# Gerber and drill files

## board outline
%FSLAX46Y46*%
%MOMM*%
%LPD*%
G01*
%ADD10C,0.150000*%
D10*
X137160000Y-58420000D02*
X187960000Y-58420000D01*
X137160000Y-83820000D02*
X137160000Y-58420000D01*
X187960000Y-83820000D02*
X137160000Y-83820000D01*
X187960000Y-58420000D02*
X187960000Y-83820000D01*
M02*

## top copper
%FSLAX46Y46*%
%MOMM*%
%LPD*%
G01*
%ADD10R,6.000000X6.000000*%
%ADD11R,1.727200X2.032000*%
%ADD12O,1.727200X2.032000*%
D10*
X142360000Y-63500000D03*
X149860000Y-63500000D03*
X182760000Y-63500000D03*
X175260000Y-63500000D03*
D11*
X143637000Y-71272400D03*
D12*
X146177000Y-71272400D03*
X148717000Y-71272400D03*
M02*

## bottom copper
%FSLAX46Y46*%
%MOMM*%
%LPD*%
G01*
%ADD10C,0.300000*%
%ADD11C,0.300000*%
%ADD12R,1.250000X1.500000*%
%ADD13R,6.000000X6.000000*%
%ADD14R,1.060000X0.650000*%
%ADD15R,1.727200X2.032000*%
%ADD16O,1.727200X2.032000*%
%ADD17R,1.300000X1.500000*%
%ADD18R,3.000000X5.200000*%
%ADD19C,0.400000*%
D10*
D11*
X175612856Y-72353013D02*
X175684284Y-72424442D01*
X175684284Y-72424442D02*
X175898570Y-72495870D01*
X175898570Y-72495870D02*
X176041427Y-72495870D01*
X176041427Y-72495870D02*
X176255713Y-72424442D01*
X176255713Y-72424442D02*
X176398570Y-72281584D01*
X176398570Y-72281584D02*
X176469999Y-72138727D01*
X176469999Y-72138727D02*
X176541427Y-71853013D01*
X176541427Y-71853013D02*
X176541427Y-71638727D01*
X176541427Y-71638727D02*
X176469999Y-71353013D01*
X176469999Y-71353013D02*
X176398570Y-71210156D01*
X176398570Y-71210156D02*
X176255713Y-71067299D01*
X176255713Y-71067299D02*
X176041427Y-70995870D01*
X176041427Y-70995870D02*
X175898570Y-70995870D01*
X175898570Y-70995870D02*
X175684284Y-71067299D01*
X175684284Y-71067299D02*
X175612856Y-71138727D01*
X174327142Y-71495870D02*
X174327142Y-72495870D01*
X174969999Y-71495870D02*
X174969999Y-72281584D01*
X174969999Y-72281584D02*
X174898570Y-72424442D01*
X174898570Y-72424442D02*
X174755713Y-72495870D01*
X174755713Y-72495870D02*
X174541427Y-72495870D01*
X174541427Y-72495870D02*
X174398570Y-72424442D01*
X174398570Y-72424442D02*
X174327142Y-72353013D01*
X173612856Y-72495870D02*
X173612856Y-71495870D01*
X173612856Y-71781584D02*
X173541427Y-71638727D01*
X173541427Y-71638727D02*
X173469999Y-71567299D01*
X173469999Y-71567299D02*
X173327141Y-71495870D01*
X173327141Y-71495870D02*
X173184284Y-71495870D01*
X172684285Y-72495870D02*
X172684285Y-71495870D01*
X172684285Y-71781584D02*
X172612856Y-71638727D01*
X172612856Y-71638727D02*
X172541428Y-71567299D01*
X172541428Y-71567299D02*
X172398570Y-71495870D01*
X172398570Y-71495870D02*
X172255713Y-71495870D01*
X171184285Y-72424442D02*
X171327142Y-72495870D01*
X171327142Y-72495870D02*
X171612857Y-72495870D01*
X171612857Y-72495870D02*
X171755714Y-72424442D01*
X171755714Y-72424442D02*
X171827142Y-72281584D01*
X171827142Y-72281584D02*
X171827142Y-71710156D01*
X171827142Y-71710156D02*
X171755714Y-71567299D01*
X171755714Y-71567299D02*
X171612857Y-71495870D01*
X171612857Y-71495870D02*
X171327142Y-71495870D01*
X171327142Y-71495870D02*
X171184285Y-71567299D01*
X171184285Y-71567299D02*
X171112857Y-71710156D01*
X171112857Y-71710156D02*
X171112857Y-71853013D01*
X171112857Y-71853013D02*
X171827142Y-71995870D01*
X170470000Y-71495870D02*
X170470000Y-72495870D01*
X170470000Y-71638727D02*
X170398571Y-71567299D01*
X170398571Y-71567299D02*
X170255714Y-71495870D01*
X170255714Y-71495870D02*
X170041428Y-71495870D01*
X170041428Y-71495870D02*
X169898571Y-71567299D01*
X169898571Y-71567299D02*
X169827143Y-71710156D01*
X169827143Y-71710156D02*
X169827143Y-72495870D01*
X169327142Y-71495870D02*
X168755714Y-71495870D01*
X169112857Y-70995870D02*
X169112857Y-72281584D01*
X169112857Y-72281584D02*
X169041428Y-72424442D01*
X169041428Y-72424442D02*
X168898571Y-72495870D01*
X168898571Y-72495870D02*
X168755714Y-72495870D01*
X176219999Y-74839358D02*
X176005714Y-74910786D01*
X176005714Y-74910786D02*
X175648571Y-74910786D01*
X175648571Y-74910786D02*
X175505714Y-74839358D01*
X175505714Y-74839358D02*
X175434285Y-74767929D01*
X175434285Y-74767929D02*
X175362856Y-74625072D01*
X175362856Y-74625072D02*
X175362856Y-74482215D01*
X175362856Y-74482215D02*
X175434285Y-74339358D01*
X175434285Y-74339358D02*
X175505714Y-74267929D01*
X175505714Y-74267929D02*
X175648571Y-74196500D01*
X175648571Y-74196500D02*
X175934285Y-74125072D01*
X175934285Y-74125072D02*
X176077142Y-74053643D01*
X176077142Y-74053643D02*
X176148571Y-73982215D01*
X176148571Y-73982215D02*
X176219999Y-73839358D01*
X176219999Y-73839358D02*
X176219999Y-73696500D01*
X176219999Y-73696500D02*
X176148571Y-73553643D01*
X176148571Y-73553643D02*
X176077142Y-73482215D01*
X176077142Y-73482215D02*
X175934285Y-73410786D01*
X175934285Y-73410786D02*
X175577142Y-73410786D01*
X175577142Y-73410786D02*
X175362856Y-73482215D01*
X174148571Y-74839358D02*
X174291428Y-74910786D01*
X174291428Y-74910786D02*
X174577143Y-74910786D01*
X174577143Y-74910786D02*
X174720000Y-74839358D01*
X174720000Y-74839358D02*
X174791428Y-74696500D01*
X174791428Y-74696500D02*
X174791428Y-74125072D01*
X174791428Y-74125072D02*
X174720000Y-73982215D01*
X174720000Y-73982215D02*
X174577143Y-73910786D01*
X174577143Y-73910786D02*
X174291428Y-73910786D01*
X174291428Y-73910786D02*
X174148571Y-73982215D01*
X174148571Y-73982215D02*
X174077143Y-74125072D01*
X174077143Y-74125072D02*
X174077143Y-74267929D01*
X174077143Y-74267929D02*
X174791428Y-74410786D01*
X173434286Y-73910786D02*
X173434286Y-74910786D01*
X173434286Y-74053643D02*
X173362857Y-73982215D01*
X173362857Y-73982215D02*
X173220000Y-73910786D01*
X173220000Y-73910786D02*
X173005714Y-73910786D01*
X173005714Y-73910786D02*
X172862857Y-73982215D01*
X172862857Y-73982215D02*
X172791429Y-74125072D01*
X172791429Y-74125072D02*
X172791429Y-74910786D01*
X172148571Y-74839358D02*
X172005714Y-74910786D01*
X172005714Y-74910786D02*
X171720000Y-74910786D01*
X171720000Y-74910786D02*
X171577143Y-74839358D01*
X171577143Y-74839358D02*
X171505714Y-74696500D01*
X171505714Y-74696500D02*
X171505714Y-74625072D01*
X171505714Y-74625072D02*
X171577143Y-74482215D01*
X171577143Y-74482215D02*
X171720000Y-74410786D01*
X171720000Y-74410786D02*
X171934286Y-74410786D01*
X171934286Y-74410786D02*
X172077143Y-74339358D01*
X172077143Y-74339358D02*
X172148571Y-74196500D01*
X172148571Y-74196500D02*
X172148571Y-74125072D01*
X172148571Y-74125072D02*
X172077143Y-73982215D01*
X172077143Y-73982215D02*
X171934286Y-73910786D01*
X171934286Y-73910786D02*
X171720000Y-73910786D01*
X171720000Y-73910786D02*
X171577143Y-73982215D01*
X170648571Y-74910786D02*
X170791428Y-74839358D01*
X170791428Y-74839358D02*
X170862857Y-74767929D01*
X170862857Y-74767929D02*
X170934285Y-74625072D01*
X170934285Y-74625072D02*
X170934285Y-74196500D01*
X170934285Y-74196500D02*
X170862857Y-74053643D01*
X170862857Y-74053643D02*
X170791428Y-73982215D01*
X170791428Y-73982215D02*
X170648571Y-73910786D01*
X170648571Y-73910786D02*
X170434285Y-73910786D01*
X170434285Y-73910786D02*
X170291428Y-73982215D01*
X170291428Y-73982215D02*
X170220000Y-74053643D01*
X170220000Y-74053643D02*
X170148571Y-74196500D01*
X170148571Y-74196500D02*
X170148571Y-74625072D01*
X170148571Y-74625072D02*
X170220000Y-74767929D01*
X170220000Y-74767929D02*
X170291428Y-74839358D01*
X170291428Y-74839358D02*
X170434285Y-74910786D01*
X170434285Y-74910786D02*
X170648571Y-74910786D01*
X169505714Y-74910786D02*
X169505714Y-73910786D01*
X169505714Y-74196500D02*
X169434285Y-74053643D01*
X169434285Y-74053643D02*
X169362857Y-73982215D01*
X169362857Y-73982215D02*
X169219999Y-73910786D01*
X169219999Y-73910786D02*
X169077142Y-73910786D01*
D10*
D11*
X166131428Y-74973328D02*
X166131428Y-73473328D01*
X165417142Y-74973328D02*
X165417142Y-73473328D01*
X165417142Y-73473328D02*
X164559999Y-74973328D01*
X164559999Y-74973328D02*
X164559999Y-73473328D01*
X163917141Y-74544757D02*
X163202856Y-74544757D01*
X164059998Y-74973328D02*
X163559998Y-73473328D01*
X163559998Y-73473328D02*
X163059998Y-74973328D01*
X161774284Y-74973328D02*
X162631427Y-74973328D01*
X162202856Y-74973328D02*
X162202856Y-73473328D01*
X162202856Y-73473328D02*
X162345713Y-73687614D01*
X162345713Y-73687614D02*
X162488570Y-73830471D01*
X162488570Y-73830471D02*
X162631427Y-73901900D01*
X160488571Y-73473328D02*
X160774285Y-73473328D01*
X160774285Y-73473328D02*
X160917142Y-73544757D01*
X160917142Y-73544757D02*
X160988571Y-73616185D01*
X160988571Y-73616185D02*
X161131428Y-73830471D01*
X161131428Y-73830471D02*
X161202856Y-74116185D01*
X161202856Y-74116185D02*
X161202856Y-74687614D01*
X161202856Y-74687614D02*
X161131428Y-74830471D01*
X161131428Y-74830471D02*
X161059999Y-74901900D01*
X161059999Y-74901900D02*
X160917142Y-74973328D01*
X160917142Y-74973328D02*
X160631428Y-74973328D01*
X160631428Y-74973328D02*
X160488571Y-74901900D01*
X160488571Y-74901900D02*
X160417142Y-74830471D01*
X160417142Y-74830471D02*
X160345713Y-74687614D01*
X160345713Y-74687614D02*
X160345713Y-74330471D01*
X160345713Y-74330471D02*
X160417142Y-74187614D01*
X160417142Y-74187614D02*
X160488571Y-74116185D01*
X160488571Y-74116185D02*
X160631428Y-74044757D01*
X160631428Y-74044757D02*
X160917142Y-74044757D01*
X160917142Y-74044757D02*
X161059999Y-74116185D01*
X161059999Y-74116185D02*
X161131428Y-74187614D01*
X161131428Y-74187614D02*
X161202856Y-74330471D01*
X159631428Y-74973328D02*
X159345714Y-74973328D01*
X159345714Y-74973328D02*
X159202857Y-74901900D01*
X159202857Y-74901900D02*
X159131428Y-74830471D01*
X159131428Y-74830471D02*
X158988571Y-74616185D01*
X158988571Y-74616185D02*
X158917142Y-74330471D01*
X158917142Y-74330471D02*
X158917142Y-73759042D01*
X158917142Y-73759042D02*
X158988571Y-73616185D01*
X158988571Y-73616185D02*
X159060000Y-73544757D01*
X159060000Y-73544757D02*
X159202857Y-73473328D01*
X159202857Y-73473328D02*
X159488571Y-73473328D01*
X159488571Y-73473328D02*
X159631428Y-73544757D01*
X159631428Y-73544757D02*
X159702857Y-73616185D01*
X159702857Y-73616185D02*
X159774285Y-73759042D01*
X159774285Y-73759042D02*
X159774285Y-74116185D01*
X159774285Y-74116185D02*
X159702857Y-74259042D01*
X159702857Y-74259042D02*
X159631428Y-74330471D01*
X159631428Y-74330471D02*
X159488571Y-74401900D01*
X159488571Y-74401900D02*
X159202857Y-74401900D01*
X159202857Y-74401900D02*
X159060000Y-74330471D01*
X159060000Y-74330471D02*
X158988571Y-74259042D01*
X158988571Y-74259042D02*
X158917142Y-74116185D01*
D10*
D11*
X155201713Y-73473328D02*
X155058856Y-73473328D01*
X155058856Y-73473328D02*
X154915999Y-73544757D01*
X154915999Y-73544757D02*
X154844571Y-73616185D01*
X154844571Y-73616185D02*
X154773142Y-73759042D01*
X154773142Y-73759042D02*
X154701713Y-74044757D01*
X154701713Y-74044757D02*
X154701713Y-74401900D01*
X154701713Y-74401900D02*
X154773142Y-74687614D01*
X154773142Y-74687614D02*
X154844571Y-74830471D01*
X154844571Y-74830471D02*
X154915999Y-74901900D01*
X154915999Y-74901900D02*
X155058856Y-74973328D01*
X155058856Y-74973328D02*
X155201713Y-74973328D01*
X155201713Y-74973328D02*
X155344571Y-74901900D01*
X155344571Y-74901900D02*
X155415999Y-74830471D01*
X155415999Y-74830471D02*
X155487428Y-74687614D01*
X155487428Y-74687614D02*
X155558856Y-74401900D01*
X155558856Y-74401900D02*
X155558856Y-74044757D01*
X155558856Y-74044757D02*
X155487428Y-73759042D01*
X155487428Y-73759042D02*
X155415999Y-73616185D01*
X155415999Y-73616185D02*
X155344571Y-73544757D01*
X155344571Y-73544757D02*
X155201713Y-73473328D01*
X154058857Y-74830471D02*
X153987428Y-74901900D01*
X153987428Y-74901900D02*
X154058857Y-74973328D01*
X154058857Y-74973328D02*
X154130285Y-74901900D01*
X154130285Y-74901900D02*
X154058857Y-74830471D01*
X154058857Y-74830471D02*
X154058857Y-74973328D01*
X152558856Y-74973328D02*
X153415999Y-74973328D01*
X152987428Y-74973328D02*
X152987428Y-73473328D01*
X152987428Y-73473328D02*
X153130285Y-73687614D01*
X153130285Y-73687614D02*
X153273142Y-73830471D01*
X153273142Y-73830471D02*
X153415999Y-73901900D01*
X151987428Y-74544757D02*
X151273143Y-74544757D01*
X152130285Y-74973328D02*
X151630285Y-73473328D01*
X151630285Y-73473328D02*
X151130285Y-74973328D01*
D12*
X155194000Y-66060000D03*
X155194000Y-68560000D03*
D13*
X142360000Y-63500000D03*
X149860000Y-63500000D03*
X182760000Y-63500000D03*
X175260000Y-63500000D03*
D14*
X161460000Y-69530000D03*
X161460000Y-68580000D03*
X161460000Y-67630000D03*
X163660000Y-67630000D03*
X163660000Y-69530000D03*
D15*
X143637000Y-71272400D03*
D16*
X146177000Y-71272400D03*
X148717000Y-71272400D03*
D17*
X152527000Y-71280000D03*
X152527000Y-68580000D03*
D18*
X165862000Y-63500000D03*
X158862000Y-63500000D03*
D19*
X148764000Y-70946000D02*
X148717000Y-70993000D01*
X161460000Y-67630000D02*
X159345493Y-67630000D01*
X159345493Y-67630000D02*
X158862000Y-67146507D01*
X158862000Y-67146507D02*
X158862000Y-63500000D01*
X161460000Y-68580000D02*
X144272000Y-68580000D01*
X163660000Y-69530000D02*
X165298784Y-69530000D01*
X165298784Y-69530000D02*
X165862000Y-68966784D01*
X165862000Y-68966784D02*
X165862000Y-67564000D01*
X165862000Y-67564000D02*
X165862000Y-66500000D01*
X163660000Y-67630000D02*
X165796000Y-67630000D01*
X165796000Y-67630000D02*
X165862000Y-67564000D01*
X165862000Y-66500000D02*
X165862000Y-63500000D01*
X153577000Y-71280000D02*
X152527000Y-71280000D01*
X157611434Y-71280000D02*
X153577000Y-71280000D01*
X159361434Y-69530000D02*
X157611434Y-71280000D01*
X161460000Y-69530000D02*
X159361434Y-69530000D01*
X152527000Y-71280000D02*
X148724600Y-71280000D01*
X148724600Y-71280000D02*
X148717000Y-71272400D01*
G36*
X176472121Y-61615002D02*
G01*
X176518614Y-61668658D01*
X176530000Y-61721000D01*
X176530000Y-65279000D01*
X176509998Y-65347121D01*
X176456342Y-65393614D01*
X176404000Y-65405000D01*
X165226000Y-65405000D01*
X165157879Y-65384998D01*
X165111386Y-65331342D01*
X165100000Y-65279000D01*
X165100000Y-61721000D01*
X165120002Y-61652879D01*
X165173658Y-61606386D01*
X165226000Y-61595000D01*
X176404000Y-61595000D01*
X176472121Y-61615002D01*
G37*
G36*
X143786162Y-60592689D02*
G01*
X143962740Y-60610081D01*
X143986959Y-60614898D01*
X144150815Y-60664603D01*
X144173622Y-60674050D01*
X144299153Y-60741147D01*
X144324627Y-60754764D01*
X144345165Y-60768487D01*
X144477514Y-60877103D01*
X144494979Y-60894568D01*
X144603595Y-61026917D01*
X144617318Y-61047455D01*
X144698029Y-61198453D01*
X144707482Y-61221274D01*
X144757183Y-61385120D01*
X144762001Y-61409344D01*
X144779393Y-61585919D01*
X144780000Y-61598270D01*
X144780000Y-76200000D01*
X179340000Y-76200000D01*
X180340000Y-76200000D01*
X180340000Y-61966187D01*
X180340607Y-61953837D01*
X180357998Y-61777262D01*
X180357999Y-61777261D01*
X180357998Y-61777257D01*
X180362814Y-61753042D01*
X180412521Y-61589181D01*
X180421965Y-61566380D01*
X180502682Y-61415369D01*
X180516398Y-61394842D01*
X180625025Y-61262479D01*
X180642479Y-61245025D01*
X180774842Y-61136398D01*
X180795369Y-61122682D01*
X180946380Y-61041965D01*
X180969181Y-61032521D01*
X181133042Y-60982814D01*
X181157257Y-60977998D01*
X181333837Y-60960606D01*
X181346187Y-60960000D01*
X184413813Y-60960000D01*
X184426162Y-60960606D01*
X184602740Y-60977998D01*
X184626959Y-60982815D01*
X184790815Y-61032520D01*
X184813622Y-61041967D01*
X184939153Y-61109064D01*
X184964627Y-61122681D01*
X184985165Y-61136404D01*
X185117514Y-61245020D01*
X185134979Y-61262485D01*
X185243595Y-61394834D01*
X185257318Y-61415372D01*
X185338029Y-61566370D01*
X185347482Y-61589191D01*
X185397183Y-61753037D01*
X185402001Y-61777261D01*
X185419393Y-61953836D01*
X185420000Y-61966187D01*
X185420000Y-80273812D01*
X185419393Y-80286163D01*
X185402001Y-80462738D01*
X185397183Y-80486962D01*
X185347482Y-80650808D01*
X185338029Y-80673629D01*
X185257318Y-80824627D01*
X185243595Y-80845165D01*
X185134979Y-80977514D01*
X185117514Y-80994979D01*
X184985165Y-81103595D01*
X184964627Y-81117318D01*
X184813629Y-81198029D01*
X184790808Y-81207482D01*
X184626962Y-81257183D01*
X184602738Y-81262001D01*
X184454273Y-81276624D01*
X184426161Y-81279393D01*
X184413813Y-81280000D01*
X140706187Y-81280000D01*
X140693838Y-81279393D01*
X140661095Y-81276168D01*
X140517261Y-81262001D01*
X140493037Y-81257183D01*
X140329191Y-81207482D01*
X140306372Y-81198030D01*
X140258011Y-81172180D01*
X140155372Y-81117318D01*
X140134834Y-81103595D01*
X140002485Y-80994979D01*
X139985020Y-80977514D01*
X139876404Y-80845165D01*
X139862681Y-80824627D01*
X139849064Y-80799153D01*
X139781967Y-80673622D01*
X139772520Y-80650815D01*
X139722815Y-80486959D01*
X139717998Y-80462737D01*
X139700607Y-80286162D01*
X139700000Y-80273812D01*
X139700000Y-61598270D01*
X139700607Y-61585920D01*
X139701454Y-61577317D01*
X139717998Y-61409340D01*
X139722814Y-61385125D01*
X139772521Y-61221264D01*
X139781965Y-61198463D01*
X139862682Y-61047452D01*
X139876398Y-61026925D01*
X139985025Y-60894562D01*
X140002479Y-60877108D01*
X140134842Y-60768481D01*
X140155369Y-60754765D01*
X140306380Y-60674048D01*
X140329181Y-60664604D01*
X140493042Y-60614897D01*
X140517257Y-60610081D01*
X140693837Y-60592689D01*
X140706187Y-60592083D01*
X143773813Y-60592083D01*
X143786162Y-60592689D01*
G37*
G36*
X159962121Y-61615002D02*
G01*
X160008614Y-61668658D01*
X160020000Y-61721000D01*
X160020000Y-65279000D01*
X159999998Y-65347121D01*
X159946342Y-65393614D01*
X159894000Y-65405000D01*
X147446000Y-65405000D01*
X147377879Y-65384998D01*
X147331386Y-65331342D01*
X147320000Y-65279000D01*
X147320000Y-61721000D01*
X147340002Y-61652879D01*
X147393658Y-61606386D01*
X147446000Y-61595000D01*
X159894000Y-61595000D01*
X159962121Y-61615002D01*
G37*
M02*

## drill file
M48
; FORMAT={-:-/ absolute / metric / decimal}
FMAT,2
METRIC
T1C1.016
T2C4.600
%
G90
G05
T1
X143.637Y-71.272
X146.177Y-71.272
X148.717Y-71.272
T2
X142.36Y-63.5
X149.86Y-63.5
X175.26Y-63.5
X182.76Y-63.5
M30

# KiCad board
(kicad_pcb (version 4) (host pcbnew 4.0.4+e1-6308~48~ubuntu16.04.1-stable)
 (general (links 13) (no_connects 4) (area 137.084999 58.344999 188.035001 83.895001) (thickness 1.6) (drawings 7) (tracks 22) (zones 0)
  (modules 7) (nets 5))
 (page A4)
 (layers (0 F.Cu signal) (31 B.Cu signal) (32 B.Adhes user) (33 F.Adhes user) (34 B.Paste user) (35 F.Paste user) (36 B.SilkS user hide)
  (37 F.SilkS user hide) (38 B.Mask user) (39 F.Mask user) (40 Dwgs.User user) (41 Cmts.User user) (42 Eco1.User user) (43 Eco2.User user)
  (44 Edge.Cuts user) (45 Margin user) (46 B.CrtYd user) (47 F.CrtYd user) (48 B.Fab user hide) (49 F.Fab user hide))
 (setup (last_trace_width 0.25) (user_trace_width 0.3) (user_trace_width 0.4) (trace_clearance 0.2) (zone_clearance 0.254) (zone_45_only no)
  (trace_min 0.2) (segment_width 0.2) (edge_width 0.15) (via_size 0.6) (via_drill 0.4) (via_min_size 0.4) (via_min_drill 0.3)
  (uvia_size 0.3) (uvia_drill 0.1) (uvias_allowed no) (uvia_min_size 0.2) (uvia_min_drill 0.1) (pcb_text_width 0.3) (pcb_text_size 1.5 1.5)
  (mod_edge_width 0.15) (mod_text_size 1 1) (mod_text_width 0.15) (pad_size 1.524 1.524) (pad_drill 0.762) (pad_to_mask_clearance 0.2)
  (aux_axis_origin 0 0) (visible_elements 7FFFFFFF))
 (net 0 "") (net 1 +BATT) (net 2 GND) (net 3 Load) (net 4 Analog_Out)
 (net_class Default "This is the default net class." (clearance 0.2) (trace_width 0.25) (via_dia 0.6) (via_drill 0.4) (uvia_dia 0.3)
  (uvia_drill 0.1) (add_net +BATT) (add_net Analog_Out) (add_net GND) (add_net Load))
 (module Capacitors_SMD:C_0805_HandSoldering (layer B.Cu) (at 155.194 67.31 270)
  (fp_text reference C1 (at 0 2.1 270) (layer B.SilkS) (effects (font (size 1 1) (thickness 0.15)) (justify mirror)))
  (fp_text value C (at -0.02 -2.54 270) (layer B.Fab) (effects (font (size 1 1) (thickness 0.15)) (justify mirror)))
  (pad 1 smd rect (at -1.25 0 270) (size 1.5 1.25) (layers B.Cu B.Paste B.Mask) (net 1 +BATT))
  (pad 2 smd rect (at 1.25 0 270) (size 1.5 1.25) (layers B.Cu B.Paste B.Mask) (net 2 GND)))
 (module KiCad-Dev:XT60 (layer F.Cu) (at 142.36 63.5)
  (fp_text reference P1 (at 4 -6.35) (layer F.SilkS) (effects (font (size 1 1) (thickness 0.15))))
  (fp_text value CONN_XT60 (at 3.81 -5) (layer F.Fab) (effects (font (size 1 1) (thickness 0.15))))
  (pad 1 thru_hole rect (at 0 0) (size 6 6) (drill 4.6) (layers *.Cu *.Mask) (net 2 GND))
  (pad 2 thru_hole rect (at 7.5 0) (size 6 6) (drill 4.6) (layers *.Cu *.Mask) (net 1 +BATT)))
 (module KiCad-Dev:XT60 (layer F.Cu) (at 182.76 63.5 180)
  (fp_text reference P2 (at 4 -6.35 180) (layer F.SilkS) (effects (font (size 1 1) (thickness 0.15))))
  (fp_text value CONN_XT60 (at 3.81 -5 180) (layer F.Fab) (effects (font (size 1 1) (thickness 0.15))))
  (pad 1 thru_hole rect (at 0 0 180) (size 6 6) (drill 4.6) (layers *.Cu *.Mask) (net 2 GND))
  (pad 2 thru_hole rect (at 7.5 0 180) (size 6 6) (drill 4.6) (layers *.Cu *.Mask) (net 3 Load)))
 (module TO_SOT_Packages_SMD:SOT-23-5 (layer B.Cu) (at 162.56 68.58)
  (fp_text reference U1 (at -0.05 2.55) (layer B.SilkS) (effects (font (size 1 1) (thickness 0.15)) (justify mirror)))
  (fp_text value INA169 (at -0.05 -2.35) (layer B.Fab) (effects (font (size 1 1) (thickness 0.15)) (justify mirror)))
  (pad 1 smd rect (at -1.1 0.95) (size 1.06 0.65) (layers B.Cu B.Paste B.Mask) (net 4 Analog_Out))
  (pad 2 smd rect (at -1.1 0) (size 1.06 0.65) (layers B.Cu B.Paste B.Mask) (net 2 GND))
  (pad 3 smd rect (at -1.1 -0.95) (size 1.06 0.65) (layers B.Cu B.Paste B.Mask) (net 1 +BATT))
  (pad 4 smd rect (at 1.1 -0.95) (size 1.06 0.65) (layers B.Cu B.Paste B.Mask) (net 3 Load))
  (pad 5 smd rect (at 1.1 0.95) (size 1.06 0.65) (layers B.Cu B.Paste B.Mask) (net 3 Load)))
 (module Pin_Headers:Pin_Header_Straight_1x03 (layer F.Cu) (at 143.637 71.2724 90)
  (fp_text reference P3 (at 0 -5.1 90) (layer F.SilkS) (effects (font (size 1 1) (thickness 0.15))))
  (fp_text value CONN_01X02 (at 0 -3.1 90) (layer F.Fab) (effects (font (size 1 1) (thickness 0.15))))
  (pad 1 thru_hole rect (at 0 0 90) (size 2.032 1.7272) (drill 1.016) (layers *.Cu *.Mask F.SilkS) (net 2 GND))
  (pad 2 thru_hole oval (at 0 2.54 90) (size 2.032 1.7272) (drill 1.016) (layers *.Cu *.Mask F.SilkS) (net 4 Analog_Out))
  (pad 3 thru_hole oval (at 0 5.08 90) (size 2.032 1.7272) (drill 1.016) (layers *.Cu *.Mask F.SilkS)))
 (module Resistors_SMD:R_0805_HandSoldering (layer B.Cu) (at 152.527 69.93 90)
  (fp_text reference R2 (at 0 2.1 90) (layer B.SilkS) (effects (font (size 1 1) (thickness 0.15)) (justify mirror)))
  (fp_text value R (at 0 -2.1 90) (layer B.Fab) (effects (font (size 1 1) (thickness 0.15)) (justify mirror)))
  (pad 1 smd rect (at -1.35 0 90) (size 1.5 1.3) (layers B.Cu B.Paste B.Mask) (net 4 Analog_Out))
  (pad 2 smd rect (at 1.35 0 90) (size 1.5 1.3) (layers B.Cu B.Paste B.Mask) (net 2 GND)))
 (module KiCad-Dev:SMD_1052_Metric (layer B.Cu) (at 167.362 60.9 180)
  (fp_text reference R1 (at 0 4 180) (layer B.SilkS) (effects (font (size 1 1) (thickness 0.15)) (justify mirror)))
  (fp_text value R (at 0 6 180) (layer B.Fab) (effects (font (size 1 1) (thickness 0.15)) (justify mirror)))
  (pad 1 smd rect (at 1.5 -2.6 180) (size 3 5.2) (layers B.Cu B.Paste B.Mask) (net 3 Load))
  (pad 2 smd rect (at 8.5 -2.6 180) (size 3 5.2) (layers B.Cu B.Paste B.Mask) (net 1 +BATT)))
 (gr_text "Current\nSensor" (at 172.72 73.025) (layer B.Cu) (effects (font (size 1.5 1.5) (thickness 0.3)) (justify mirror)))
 (gr_line (start 137.16 58.42) (end 187.96 58.42) (layer Edge.Cuts) (width 0.15))
 (gr_line (start 137.16 83.82) (end 137.16 58.42) (layer Edge.Cuts) (width 0.15))
 (gr_line (start 187.96 83.82) (end 137.16 83.82) (layer Edge.Cuts) (width 0.15))
 (gr_line (start 187.96 58.42) (end 187.96 83.82) (layer Edge.Cuts) (width 0.15))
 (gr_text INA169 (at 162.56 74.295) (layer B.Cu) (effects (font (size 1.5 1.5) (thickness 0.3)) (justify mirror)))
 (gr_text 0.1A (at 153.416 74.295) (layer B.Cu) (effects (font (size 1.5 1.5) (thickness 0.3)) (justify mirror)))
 (segment (start 187.96 58.42) (end 137.16 58.42) (width 0.4) (layer Dwgs.User) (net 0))
 (segment (start 187.96 83.82) (end 187.96 58.42) (width 0.4) (layer Dwgs.User) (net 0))
 (segment (start 137.16 83.82) (end 187.96 83.82) (width 0.4) (layer Dwgs.User) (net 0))
 (segment (start 137.16 58.42) (end 137.16 83.82) (width 0.4) (layer Dwgs.User) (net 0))
 (segment (start 148.764 70.946) (end 148.717 70.993) (width 0.4) (layer B.Cu) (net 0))
 (segment (start 161.46 67.63) (end 159.345493 67.63) (width 0.4) (layer B.Cu) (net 1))
 (segment (start 159.345493 67.63) (end 158.862 67.146507) (width 0.4) (layer B.Cu) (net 1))
 (segment (start 158.862 67.146507) (end 158.862 63.5) (width 0.4) (layer B.Cu) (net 1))
 (segment (start 161.46 68.58) (end 144.272 68.58) (width 0.4) (layer B.Cu) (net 2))
 (segment (start 163.66 69.53) (end 165.298784 69.53) (width 0.4) (layer B.Cu) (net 3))
 (segment (start 165.298784 69.53) (end 165.862 68.966784) (width 0.4) (layer B.Cu) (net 3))
 (segment (start 165.862 68.966784) (end 165.862 67.564) (width 0.4) (layer B.Cu) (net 3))
 (segment (start 165.862 67.564) (end 165.862 66.5) (width 0.4) (layer B.Cu) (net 3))
 (segment (start 163.66 67.63) (end 165.796 67.63) (width 0.4) (layer B.Cu) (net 3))
 (segment (start 165.796 67.63) (end 165.862 67.564) (width 0.4) (layer B.Cu) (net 3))
 (segment (start 165.862 66.5) (end 165.862 63.5) (width 0.4) (layer B.Cu) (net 3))
 (segment (start 153.577 71.28) (end 152.527 71.28) (width 0.4) (layer B.Cu) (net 4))
 (segment (start 157.611434 71.28) (end 153.577 71.28) (width 0.4) (layer B.Cu) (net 4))
 (segment (start 159.361434 69.53) (end 157.611434 71.28) (width 0.4) (layer B.Cu) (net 4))
 (segment (start 161.46 69.53) (end 159.361434 69.53) (width 0.4) (layer B.Cu) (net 4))
 (segment (start 152.527 71.28) (end 148.7246 71.28) (width 0.4) (layer B.Cu) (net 4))
 (segment (start 148.7246 71.28) (end 148.717 71.2724) (width 0.4) (layer B.Cu) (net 4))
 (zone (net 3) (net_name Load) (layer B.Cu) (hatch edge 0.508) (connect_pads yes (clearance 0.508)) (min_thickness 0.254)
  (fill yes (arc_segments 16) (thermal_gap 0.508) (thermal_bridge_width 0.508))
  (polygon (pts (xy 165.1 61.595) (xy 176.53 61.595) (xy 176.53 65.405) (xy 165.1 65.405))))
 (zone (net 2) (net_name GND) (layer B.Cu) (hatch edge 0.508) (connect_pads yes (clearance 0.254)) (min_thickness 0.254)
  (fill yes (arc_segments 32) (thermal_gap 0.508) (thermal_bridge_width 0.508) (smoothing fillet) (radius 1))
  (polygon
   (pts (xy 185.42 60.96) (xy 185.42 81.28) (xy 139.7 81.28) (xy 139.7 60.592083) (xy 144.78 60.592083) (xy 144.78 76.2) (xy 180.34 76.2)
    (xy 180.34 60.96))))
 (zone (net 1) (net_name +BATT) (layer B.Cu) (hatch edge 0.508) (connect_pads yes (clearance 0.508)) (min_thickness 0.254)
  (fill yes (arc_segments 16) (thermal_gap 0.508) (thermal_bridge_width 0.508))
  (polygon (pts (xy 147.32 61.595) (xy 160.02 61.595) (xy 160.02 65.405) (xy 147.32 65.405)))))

